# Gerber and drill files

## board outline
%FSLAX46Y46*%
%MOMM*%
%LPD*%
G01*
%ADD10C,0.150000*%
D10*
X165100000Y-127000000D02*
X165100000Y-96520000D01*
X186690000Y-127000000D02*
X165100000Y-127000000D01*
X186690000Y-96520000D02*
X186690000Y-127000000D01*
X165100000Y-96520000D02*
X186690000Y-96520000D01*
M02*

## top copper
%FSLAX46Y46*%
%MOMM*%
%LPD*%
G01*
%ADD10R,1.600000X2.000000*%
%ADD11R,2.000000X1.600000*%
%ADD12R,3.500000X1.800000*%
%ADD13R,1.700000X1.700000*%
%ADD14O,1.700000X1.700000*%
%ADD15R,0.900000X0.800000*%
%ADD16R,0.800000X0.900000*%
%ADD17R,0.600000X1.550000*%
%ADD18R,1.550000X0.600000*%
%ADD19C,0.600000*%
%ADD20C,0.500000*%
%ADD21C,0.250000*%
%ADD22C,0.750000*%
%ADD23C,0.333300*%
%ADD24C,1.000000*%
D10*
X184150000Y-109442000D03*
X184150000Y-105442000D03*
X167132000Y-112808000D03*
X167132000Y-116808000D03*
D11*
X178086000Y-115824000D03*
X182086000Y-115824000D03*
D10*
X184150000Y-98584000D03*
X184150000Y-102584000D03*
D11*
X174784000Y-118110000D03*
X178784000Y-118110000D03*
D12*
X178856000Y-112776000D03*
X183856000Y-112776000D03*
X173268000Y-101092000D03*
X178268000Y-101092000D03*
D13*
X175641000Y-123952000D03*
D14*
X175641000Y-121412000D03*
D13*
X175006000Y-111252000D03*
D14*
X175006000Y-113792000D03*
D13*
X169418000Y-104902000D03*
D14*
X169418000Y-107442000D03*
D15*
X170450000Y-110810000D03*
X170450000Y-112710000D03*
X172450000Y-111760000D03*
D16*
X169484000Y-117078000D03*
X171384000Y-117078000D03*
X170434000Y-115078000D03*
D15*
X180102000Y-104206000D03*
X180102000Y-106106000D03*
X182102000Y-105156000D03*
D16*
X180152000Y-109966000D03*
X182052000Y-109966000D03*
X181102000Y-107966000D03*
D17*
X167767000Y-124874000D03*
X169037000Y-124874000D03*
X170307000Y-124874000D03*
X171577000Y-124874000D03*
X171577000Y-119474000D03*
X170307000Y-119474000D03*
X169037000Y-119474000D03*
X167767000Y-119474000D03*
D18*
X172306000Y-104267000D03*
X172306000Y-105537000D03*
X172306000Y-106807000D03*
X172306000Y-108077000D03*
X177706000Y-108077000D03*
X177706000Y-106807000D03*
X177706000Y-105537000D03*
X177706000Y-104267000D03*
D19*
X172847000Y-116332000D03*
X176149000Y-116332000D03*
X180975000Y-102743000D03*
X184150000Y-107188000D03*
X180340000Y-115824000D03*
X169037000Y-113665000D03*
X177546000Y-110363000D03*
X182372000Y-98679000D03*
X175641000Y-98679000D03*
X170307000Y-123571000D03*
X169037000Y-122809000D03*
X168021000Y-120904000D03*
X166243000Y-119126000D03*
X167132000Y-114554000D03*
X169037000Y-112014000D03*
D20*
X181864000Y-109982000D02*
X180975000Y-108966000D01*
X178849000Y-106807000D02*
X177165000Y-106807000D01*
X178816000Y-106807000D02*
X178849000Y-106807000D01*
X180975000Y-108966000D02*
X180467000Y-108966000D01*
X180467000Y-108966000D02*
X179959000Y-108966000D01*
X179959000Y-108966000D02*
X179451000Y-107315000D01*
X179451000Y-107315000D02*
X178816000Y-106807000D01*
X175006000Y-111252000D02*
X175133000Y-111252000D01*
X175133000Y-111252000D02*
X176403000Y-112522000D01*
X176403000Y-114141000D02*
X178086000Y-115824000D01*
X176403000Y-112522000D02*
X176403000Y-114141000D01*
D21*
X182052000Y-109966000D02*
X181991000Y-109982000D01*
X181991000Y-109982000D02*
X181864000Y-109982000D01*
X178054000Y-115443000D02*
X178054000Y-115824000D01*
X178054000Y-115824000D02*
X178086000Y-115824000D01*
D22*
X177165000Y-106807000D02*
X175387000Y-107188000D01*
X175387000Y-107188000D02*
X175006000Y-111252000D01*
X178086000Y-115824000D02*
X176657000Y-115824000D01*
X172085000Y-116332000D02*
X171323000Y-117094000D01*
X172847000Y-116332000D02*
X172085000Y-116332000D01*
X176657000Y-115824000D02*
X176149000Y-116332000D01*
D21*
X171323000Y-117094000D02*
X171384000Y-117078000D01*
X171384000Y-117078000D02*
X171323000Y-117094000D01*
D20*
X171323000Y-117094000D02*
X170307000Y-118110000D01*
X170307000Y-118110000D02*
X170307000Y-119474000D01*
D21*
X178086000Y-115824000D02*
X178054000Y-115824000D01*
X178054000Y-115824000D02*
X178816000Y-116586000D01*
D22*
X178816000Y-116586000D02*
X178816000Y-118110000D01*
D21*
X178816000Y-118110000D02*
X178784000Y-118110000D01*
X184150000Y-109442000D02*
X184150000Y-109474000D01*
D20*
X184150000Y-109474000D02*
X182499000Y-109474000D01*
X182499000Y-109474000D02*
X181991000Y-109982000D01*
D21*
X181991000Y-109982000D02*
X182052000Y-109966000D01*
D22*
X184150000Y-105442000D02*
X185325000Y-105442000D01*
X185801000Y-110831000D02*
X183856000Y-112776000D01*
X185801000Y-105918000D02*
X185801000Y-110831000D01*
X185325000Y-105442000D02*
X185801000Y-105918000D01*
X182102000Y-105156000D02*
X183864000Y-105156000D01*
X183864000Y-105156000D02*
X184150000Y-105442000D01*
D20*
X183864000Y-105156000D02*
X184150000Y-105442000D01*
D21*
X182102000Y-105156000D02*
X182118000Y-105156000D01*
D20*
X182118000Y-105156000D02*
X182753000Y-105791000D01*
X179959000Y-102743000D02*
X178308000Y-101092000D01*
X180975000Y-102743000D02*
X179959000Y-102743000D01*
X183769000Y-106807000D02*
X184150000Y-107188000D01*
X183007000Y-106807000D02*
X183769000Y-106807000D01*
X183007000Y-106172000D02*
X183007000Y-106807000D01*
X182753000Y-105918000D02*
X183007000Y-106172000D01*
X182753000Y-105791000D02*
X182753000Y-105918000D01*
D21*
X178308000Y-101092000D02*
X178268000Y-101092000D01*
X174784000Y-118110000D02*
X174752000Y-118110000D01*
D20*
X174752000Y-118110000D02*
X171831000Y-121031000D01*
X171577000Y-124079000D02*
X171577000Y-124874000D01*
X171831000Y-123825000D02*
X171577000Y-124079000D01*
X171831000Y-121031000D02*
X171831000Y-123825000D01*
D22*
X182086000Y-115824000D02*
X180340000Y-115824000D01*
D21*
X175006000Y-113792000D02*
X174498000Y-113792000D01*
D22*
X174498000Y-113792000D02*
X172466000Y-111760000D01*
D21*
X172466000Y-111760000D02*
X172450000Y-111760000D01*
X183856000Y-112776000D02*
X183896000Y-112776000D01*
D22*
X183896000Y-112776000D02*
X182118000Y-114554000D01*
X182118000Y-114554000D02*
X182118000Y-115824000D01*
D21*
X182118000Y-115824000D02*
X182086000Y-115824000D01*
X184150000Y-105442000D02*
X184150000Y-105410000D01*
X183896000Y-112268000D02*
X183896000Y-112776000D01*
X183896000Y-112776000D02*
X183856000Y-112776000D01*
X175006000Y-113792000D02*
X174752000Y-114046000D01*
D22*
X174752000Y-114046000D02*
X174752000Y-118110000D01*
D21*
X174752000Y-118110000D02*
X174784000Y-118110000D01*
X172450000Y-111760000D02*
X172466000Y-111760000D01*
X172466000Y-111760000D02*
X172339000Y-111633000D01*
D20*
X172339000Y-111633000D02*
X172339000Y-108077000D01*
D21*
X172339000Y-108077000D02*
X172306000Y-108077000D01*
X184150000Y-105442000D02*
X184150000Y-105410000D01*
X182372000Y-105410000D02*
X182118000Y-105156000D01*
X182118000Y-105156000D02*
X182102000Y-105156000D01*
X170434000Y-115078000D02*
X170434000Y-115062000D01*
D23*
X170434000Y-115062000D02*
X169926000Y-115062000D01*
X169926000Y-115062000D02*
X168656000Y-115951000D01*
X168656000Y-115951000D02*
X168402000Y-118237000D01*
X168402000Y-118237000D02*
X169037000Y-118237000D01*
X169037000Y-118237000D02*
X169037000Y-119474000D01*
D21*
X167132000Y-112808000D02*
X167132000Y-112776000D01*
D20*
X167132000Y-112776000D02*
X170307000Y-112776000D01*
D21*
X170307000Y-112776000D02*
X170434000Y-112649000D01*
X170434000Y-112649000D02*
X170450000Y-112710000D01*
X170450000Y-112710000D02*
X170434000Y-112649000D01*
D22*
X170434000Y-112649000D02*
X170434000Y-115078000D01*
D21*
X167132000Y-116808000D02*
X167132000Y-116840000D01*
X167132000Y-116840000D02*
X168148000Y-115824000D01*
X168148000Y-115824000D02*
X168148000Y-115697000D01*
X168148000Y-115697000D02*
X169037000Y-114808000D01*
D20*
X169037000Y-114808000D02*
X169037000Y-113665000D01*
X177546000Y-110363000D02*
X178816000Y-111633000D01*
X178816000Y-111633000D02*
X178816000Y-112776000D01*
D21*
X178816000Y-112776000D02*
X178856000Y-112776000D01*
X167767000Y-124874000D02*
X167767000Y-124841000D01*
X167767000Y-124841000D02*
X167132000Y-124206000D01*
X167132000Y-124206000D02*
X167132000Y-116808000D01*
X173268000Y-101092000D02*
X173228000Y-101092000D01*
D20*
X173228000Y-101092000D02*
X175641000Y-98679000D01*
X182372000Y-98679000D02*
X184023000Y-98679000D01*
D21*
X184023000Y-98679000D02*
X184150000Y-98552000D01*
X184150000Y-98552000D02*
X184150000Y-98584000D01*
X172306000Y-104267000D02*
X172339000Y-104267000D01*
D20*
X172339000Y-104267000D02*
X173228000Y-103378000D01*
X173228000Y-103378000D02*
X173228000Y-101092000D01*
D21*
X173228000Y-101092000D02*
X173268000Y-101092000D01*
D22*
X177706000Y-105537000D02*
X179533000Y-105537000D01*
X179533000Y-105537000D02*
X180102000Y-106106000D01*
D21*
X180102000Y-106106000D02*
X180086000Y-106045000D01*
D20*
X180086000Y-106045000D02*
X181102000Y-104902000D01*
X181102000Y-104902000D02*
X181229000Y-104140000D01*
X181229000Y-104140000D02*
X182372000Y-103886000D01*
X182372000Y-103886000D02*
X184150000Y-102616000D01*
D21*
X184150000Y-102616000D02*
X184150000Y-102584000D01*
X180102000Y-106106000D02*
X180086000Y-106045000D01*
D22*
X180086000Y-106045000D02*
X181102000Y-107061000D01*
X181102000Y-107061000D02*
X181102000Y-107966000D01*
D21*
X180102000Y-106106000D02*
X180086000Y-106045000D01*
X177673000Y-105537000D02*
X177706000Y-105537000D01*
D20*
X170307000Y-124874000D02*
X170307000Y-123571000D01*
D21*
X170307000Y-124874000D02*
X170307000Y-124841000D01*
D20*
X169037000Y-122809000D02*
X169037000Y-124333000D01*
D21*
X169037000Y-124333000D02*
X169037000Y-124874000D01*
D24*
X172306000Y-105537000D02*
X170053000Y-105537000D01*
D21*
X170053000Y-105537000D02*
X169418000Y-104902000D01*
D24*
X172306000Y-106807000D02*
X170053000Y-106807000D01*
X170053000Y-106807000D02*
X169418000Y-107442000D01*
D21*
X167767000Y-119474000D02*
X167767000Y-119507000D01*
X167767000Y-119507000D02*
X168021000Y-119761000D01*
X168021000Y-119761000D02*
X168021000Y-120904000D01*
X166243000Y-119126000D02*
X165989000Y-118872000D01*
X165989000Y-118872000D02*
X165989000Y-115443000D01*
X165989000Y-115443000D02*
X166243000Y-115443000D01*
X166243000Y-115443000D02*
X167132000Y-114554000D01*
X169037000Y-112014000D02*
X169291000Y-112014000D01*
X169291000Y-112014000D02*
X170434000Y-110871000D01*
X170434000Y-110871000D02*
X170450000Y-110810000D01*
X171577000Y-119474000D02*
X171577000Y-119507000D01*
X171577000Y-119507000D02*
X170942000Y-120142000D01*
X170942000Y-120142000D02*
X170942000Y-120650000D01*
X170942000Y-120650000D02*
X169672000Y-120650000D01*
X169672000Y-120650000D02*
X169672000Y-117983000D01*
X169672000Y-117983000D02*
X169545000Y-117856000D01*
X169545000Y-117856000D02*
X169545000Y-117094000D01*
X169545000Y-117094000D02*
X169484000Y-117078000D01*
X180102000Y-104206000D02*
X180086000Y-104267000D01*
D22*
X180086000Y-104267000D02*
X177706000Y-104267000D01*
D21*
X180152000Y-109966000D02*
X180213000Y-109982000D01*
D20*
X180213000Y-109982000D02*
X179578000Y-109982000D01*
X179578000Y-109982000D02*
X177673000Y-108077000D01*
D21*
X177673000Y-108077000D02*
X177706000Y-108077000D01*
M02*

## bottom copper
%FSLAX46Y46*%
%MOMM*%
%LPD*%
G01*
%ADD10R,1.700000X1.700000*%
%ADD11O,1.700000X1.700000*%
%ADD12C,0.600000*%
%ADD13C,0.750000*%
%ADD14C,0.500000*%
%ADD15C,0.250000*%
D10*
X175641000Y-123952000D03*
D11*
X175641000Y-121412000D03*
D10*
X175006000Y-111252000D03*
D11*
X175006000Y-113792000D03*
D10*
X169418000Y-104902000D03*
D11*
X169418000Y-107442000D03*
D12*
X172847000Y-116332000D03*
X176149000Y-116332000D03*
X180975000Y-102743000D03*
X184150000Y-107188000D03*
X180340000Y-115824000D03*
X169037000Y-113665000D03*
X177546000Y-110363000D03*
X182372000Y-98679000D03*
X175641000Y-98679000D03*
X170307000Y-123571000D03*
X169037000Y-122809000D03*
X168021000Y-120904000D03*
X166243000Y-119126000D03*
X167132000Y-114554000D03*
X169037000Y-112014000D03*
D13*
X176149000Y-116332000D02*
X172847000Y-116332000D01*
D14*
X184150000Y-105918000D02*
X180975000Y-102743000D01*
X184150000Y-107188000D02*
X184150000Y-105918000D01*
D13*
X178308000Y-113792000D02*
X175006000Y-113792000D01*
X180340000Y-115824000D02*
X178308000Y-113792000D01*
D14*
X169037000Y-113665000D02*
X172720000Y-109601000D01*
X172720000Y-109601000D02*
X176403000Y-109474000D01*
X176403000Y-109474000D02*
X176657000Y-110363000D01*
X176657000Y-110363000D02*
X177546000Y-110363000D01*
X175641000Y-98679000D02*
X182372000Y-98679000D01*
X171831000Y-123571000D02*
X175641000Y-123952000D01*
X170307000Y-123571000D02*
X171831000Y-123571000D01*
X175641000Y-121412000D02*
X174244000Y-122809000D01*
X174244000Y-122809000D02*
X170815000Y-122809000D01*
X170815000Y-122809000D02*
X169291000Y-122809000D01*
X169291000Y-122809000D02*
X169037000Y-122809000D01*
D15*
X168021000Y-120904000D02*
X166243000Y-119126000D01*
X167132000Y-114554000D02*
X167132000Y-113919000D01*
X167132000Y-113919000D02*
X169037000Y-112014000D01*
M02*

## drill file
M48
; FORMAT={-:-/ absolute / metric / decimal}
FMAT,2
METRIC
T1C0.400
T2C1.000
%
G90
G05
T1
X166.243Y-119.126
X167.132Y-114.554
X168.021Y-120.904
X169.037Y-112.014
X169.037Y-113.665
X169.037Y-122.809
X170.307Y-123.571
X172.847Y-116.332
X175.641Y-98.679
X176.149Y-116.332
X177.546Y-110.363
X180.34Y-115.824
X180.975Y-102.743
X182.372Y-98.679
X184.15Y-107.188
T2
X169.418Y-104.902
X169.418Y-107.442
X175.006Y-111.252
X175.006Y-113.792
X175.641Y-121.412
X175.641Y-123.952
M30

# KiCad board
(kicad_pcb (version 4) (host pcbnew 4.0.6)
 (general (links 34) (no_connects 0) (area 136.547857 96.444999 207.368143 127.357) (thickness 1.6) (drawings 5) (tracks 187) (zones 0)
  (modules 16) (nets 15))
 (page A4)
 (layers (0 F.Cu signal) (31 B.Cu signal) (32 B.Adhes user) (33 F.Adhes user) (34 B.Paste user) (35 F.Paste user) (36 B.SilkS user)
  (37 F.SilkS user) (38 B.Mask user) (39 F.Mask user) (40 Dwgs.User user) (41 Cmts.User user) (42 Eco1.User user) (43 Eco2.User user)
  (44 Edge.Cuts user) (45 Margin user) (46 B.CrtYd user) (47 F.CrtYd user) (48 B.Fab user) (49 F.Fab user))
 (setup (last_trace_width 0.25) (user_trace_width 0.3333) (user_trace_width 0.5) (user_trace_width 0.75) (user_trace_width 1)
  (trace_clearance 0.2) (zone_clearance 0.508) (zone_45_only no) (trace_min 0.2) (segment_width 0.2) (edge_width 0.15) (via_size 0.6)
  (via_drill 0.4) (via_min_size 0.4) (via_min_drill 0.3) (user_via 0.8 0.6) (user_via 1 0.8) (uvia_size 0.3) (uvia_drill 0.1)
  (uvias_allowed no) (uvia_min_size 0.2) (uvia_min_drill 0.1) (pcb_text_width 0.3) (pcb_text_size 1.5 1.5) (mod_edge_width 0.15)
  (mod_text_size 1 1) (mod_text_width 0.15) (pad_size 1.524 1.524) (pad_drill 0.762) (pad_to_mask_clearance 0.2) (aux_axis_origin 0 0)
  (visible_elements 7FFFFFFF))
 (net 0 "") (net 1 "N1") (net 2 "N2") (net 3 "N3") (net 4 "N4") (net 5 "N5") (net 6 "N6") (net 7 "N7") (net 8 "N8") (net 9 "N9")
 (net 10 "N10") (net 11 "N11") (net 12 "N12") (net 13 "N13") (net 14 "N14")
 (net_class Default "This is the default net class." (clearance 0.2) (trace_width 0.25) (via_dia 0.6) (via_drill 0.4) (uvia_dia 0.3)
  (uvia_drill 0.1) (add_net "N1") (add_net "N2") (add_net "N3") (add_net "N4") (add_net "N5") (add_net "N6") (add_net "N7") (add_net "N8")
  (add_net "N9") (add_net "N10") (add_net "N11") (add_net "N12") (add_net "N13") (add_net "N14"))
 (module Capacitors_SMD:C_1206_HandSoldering (layer F.Cu) (at 184.15 107.442 90)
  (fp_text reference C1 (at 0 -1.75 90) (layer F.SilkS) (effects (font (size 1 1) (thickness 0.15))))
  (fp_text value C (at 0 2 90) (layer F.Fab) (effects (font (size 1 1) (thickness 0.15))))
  (pad 1 smd rect (at -2 0 90) (size 2 1.6) (layers F.Cu F.Paste F.Mask) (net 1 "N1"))
  (pad 2 smd rect (at 2 0 90) (size 2 1.6) (layers F.Cu F.Paste F.Mask) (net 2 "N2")))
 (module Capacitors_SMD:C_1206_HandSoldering (layer F.Cu) (at 167.132 114.808 270)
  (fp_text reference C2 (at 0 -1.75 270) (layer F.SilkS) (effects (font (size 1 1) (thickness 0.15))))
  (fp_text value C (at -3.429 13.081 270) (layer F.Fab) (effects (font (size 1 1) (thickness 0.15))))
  (pad 1 smd rect (at -2 0 270) (size 2 1.6) (layers F.Cu F.Paste F.Mask) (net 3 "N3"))
  (pad 2 smd rect (at 2 0 270) (size 2 1.6) (layers F.Cu F.Paste F.Mask) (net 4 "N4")))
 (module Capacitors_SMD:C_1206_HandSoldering (layer F.Cu) (at 180.086 115.824)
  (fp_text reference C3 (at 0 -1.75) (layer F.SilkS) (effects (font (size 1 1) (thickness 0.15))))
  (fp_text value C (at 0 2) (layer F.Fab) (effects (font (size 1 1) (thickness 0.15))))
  (pad 1 smd rect (at -2 0) (size 2 1.6) (layers F.Cu F.Paste F.Mask) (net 1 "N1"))
  (pad 2 smd rect (at 2 0) (size 2 1.6) (layers F.Cu F.Paste F.Mask) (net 2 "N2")))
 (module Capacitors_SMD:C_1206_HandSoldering (layer F.Cu) (at 184.15 100.584 270)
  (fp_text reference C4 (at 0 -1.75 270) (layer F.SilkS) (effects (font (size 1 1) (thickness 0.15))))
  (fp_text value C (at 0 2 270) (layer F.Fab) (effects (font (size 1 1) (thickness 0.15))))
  (pad 1 smd rect (at -2 0 270) (size 2 1.6) (layers F.Cu F.Paste F.Mask) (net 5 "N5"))
  (pad 2 smd rect (at 2 0 270) (size 2 1.6) (layers F.Cu F.Paste F.Mask) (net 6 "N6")))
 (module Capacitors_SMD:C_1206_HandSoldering (layer F.Cu) (at 176.784 118.11)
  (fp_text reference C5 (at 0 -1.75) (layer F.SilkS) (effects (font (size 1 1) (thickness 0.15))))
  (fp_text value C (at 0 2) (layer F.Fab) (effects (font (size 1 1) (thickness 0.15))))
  (pad 1 smd rect (at -2 0) (size 2 1.6) (layers F.Cu F.Paste F.Mask) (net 2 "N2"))
  (pad 2 smd rect (at 2 0) (size 2 1.6) (layers F.Cu F.Paste F.Mask) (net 1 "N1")))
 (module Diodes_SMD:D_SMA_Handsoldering (layer F.Cu) (at 181.356 112.776)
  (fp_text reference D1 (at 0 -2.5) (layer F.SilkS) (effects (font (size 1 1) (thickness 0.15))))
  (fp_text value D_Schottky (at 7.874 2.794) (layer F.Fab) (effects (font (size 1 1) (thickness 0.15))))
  (pad 1 smd rect (at -2.5 0) (size 3.5 1.8) (layers F.Cu F.Paste F.Mask) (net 4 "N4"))
  (pad 2 smd rect (at 2.5 0) (size 3.5 1.8) (layers F.Cu F.Paste F.Mask) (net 2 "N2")))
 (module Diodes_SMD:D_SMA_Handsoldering (layer F.Cu) (at 175.768 101.092)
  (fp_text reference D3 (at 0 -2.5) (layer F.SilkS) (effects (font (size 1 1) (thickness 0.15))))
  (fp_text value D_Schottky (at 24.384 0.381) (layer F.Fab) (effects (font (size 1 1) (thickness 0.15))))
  (pad 1 smd rect (at -2.5 0) (size 3.5 1.8) (layers F.Cu F.Paste F.Mask) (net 5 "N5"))
  (pad 2 smd rect (at 2.5 0) (size 3.5 1.8) (layers F.Cu F.Paste F.Mask) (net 2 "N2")))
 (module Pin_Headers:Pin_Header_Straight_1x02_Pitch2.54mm (layer F.Cu) (at 175.641 123.952 180)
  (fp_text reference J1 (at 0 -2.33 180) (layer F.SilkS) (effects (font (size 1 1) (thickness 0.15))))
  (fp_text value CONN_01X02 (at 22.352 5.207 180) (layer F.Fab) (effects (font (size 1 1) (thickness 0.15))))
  (pad 1 thru_hole rect (at 0 0 180) (size 1.7 1.7) (drill 1) (layers *.Cu *.Mask) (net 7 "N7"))
  (pad 2 thru_hole oval (at 0 2.54 180) (size 1.7 1.7) (drill 1) (layers *.Cu *.Mask) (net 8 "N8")))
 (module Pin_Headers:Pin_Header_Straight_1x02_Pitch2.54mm (layer F.Cu) (at 175.006 111.252)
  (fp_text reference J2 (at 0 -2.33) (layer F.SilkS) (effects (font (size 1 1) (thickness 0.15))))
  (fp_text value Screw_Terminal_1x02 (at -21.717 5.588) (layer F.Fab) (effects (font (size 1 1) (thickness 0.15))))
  (pad 1 thru_hole rect (at 0 0) (size 1.7 1.7) (drill 1) (layers *.Cu *.Mask) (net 1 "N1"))
  (pad 2 thru_hole oval (at 0 2.54) (size 1.7 1.7) (drill 1) (layers *.Cu *.Mask) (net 2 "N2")))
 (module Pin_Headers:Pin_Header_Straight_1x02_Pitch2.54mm (layer F.Cu) (at 169.418 104.902)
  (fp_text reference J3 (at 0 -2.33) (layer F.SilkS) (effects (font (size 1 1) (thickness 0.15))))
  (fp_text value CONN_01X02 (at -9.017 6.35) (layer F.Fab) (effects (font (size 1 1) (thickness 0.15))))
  (pad 1 thru_hole rect (at 0 0) (size 1.7 1.7) (drill 1) (layers *.Cu *.Mask) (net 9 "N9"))
  (pad 2 thru_hole oval (at 0 2.54) (size 1.7 1.7) (drill 1) (layers *.Cu *.Mask) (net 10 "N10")))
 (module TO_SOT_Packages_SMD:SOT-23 (layer F.Cu) (at 171.45 111.76)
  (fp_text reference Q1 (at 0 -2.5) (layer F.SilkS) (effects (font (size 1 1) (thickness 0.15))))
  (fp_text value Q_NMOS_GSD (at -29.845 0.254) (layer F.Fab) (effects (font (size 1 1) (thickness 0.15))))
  (pad 1 smd rect (at -1 -0.95) (size 0.9 0.8) (layers F.Cu F.Paste F.Mask) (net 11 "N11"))
  (pad 2 smd rect (at -1 0.95) (size 0.9 0.8) (layers F.Cu F.Paste F.Mask) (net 3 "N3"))
  (pad 3 smd rect (at 1 0) (size 0.9 0.8) (layers F.Cu F.Paste F.Mask) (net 2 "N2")))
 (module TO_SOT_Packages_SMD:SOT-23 (layer F.Cu) (at 170.434 116.078 90)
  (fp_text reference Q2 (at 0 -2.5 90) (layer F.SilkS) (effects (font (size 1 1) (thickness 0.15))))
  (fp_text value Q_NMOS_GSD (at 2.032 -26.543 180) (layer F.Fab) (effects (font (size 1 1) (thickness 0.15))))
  (pad 1 smd rect (at -1 -0.95 90) (size 0.9 0.8) (layers F.Cu F.Paste F.Mask) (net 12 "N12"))
  (pad 2 smd rect (at -1 0.95 90) (size 0.9 0.8) (layers F.Cu F.Paste F.Mask) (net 1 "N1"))
  (pad 3 smd rect (at 1 0 90) (size 0.9 0.8) (layers F.Cu F.Paste F.Mask) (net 3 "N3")))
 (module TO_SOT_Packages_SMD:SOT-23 (layer F.Cu) (at 181.102 105.156)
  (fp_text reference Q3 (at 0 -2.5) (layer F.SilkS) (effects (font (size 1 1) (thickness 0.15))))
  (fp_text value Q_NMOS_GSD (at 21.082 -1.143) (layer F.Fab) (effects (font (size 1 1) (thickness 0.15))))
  (pad 1 smd rect (at -1 -0.95) (size 0.9 0.8) (layers F.Cu F.Paste F.Mask) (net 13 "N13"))
  (pad 2 smd rect (at -1 0.95) (size 0.9 0.8) (layers F.Cu F.Paste F.Mask) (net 6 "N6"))
  (pad 3 smd rect (at 1 0) (size 0.9 0.8) (layers F.Cu F.Paste F.Mask) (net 2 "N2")))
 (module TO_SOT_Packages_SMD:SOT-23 (layer F.Cu) (at 181.102 108.966 90)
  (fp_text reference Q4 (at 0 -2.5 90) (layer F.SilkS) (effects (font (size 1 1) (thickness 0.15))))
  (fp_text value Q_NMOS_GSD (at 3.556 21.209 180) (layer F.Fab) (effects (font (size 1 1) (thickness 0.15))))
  (pad 1 smd rect (at -1 -0.95 90) (size 0.9 0.8) (layers F.Cu F.Paste F.Mask) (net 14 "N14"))
  (pad 2 smd rect (at -1 0.95 90) (size 0.9 0.8) (layers F.Cu F.Paste F.Mask) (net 1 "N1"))
  (pad 3 smd rect (at 1 0 90) (size 0.9 0.8) (layers F.Cu F.Paste F.Mask) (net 6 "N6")))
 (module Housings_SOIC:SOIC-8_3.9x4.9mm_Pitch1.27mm (layer F.Cu) (at 169.672 122.174 90)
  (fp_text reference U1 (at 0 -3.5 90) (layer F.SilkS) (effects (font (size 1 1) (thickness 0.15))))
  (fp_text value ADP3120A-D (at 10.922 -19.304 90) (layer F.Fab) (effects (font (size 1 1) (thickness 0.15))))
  (pad 1 smd rect (at -2.7 -1.905 90) (size 1.55 0.6) (layers F.Cu F.Paste F.Mask) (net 4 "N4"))
  (pad 2 smd rect (at -2.7 -0.635 90) (size 1.55 0.6) (layers F.Cu F.Paste F.Mask) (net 8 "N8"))
  (pad 3 smd rect (at -2.7 0.635 90) (size 1.55 0.6) (layers F.Cu F.Paste F.Mask) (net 7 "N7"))
  (pad 4 smd rect (at -2.7 1.905 90) (size 1.55 0.6) (layers F.Cu F.Paste F.Mask) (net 2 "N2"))
  (pad 5 smd rect (at 2.7 1.905 90) (size 1.55 0.6) (layers F.Cu F.Paste F.Mask) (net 12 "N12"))
  (pad 6 smd rect (at 2.7 0.635 90) (size 1.55 0.6) (layers F.Cu F.Paste F.Mask) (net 1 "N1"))
  (pad 7 smd rect (at 2.7 -0.635 90) (size 1.55 0.6) (layers F.Cu F.Paste F.Mask) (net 3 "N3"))
  (pad 8 smd rect (at 2.7 -1.905 90) (size 1.55 0.6) (layers F.Cu F.Paste F.Mask) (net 11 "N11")))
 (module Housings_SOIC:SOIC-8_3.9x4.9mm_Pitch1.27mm (layer F.Cu) (at 175.006 106.172)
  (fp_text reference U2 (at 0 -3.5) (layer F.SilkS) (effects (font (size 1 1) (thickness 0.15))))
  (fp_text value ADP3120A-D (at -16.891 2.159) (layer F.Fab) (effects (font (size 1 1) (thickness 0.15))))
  (pad 1 smd rect (at -2.7 -1.905) (size 1.55 0.6) (layers F.Cu F.Paste F.Mask) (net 5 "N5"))
  (pad 2 smd rect (at -2.7 -0.635) (size 1.55 0.6) (layers F.Cu F.Paste F.Mask) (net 9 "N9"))
  (pad 3 smd rect (at -2.7 0.635) (size 1.55 0.6) (layers F.Cu F.Paste F.Mask) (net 10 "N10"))
  (pad 4 smd rect (at -2.7 1.905) (size 1.55 0.6) (layers F.Cu F.Paste F.Mask) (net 2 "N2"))
  (pad 5 smd rect (at 2.7 1.905) (size 1.55 0.6) (layers F.Cu F.Paste F.Mask) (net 14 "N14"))
  (pad 6 smd rect (at 2.7 0.635) (size 1.55 0.6) (layers F.Cu F.Paste F.Mask) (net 1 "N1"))
  (pad 7 smd rect (at 2.7 -0.635) (size 1.55 0.6) (layers F.Cu F.Paste F.Mask) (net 6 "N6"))
  (pad 8 smd rect (at 2.7 -1.905) (size 1.55 0.6) (layers F.Cu F.Paste F.Mask) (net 13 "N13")))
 (gr_line (start 165.1 127) (end 165.1 96.52) (angle 90) (layer Edge.Cuts) (width 0.15))
 (gr_line (start 186.69 127) (end 165.1 127) (angle 90) (layer Edge.Cuts) (width 0.15))
 (gr_line (start 186.69 96.52) (end 186.69 127) (angle 90) (layer Edge.Cuts) (width 0.15))
 (gr_line (start 165.1 96.52) (end 186.69 96.52) (angle 90) (layer Edge.Cuts) (width 0.15))
 (segment (start 181.864 109.982) (end 180.975 108.966) (width 0.5) (layer F.Cu) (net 1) (status 80000))
 (segment (start 178.849 106.807) (end 177.165 106.807) (width 0.5) (layer F.Cu) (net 1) (status 80000))
 (segment (start 178.816 106.807) (end 178.849 106.807) (width 0.5) (layer F.Cu) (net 1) (status 80000))
 (segment (start 180.975 108.966) (end 180.467 108.966) (width 0.5) (layer F.Cu) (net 1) (status 80000))
 (segment (start 180.467 108.966) (end 179.959 108.966) (width 0.5) (layer F.Cu) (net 1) (status 80000))
 (segment (start 179.959 108.966) (end 179.451 107.315) (width 0.5) (layer F.Cu) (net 1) (status 80000))
 (segment (start 179.451 107.315) (end 178.816 106.807) (width 0.5) (layer F.Cu) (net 1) (status 80000))
 (segment (start 175.006 111.252) (end 175.133 111.252) (width 0.5) (layer F.Cu) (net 1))
 (segment (start 175.133 111.252) (end 176.403 112.522) (width 0.5) (layer F.Cu) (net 1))
 (segment (start 176.403 114.141) (end 178.086 115.824) (width 0.5) (layer F.Cu) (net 1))
 (segment (start 176.403 112.522) (end 176.403 114.141) (width 0.5) (layer F.Cu) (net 1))
 (segment (start 182.052 109.966) (end 181.991 109.982) (width 0.25) (layer F.Cu) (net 1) (status 80000))
 (segment (start 181.991 109.982) (end 181.864 109.982) (width 0.25) (layer F.Cu) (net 1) (status 80000))
 (segment (start 178.054 115.443) (end 178.054 115.824) (width 0.25) (layer F.Cu) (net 1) (status 80000))
 (segment (start 178.054 115.824) (end 178.086 115.824) (width 0.25) (layer F.Cu) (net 1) (status 80000))
 (segment (start 177.165 106.807) (end 175.387 107.188) (width 0.75) (layer F.Cu) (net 1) (status 80000))
 (segment (start 175.387 107.188) (end 175.006 111.252) (width 0.75) (layer F.Cu) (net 1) (status 80000))
 (segment (start 178.086 115.824) (end 176.657 115.824) (width 0.75) (layer F.Cu) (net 1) (status 80000))
 (segment (start 172.085 116.332) (end 171.323 117.094) (width 0.75) (layer F.Cu) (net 1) (status 80000))
 (segment (start 172.847 116.332) (end 172.085 116.332) (width 0.75) (layer F.Cu) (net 1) (status 80000))
 (via (at 172.847 116.332) (size 0.6) (drill 0.4) (layers F.Cu B.Cu) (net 1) (status 80000))
 (segment (start 176.149 116.332) (end 172.847 116.332) (width 0.75) (layer B.Cu) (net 1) (status 80000))
 (via (at 176.149 116.332) (size 0.6) (drill 0.4) (layers F.Cu B.Cu) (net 1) (status 80000))
 (segment (start 176.657 115.824) (end 176.149 116.332) (width 0.75) (layer F.Cu) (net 1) (status 80000))
 (segment (start 171.323 117.094) (end 171.384 117.078) (width 0.25) (layer F.Cu) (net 1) (status 80000))
 (segment (start 171.384 117.078) (end 171.323 117.094) (width 0.25) (layer F.Cu) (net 1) (status 80000))
 (segment (start 171.323 117.094) (end 170.307 118.11) (width 0.5) (layer F.Cu) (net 1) (status 80000))
 (segment (start 170.307 118.11) (end 170.307 119.474) (width 0.5) (layer F.Cu) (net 1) (status 80000))
 (segment (start 178.086 115.824) (end 178.054 115.824) (width 0.25) (layer F.Cu) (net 1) (status 80000))
 (segment (start 178.054 115.824) (end 178.816 116.586) (width 0.25) (layer F.Cu) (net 1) (status 80000))
 (segment (start 178.816 116.586) (end 178.816 118.11) (width 0.75) (layer F.Cu) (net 1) (status 80000))
 (segment (start 178.816 118.11) (end 178.784 118.11) (width 0.25) (layer F.Cu) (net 1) (status 80000))
 (segment (start 184.15 109.442) (end 184.15 109.474) (width 0.25) (layer F.Cu) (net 1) (status 80000))
 (segment (start 184.15 109.474) (end 182.499 109.474) (width 0.5) (layer F.Cu) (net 1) (status 80000))
 (segment (start 182.499 109.474) (end 181.991 109.982) (width 0.5) (layer F.Cu) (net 1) (status 80000))
 (segment (start 181.991 109.982) (end 182.052 109.966) (width 0.25) (layer F.Cu) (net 1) (status 80000))
 (segment (start 184.15 105.442) (end 185.325 105.442) (width 0.75) (layer F.Cu) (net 2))
 (segment (start 185.801 110.831) (end 183.856 112.776) (width 0.75) (layer F.Cu) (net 2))
 (segment (start 185.801 105.918) (end 185.801 110.831) (width 0.75) (layer F.Cu) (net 2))
 (segment (start 185.325 105.442) (end 185.801 105.918) (width 0.75) (layer F.Cu) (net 2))
 (segment (start 182.102 105.156) (end 183.864 105.156) (width 0.75) (layer F.Cu) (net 2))
 (segment (start 183.864 105.156) (end 184.15 105.442) (width 0.75) (layer F.Cu) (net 2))
 (segment (start 183.864 105.156) (end 184.15 105.442) (width 0.5) (layer F.Cu) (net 2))
 (segment (start 182.102 105.156) (end 182.118 105.156) (width 0.25) (layer F.Cu) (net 2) (status 80000))
 (segment (start 182.118 105.156) (end 182.753 105.791) (width 0.5) (layer F.Cu) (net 2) (status 80000))
 (segment (start 179.959 102.743) (end 178.308 101.092) (width 0.5) (layer F.Cu) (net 2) (status 80000))
 (segment (start 180.975 102.743) (end 179.959 102.743) (width 0.5) (layer F.Cu) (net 2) (status 80000))
 (via (at 180.975 102.743) (size 0.6) (drill 0.4) (layers F.Cu B.Cu) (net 2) (status 80000))
 (segment (start 184.15 105.918) (end 180.975 102.743) (width 0.5) (layer B.Cu) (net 2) (status 80000))
 (segment (start 184.15 107.188) (end 184.15 105.918) (width 0.5) (layer B.Cu) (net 2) (status 80000))
 (via (at 184.15 107.188) (size 0.6) (drill 0.4) (layers F.Cu B.Cu) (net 2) (status 80000))
 (segment (start 183.769 106.807) (end 184.15 107.188) (width 0.5) (layer F.Cu) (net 2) (status 80000))
 (segment (start 183.007 106.807) (end 183.769 106.807) (width 0.5) (layer F.Cu) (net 2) (status 80000))
 (segment (start 183.007 106.172) (end 183.007 106.807) (width 0.5) (layer F.Cu) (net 2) (status 80000))
 (segment (start 182.753 105.918) (end 183.007 106.172) (width 0.5) (layer F.Cu) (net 2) (status 80000))
 (segment (start 182.753 105.791) (end 182.753 105.918) (width 0.5) (layer F.Cu) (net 2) (status 80000))
 (segment (start 178.308 101.092) (end 178.268 101.092) (width 0.25) (layer F.Cu) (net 2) (status 80000))
 (segment (start 174.784 118.11) (end 174.752 118.11) (width 0.25) (layer F.Cu) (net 2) (status 80000))
 (segment (start 174.752 118.11) (end 171.831 121.031) (width 0.5) (layer F.Cu) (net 2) (status 80000))
 (segment (start 171.577 124.079) (end 171.577 124.874) (width 0.5) (layer F.Cu) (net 2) (status 80000))
 (segment (start 171.831 123.825) (end 171.577 124.079) (width 0.5) (layer F.Cu) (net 2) (status 80000))
 (segment (start 171.831 121.031) (end 171.831 123.825) (width 0.5) (layer F.Cu) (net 2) (status 80000))
 (segment (start 182.086 115.824) (end 180.34 115.824) (width 0.75) (layer F.Cu) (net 2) (status 80000))
 (segment (start 178.308 113.792) (end 175.006 113.792) (width 0.75) (layer B.Cu) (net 2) (status 80000))
 (segment (start 180.34 115.824) (end 178.308 113.792) (width 0.75) (layer B.Cu) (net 2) (status 80000))
 (via (at 180.34 115.824) (size 0.6) (drill 0.4) (layers F.Cu B.Cu) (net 2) (status 80000))
 (segment (start 175.006 113.792) (end 174.498 113.792) (width 0.25) (layer F.Cu) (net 2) (status 80000))
 (segment (start 174.498 113.792) (end 172.466 111.76) (width 0.75) (layer F.Cu) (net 2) (status 80000))
 (segment (start 172.466 111.76) (end 172.45 111.76) (width 0.25) (layer F.Cu) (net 2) (status 80000))
 (segment (start 183.856 112.776) (end 183.896 112.776) (width 0.25) (layer F.Cu) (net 2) (status 80000))
 (segment (start 183.896 112.776) (end 182.118 114.554) (width 0.75) (layer F.Cu) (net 2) (status 80000))
 (segment (start 182.118 114.554) (end 182.118 115.824) (width 0.75) (layer F.Cu) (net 2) (status 80000))
 (segment (start 182.118 115.824) (end 182.086 115.824) (width 0.25) (layer F.Cu) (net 2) (status 80000))
 (segment (start 184.15 105.442) (end 184.15 105.41) (width 0.25) (layer F.Cu) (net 2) (status 80000))
 (segment (start 183.896 112.268) (end 183.896 112.776) (width 0.25) (layer F.Cu) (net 2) (status 80000))
 (segment (start 183.896 112.776) (end 183.856 112.776) (width 0.25) (layer F.Cu) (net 2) (status 80000))
 (segment (start 175.006 113.792) (end 174.752 114.046) (width 0.25) (layer F.Cu) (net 2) (status 80000))
 (segment (start 174.752 114.046) (end 174.752 118.11) (width 0.75) (layer F.Cu) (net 2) (status 80000))
 (segment (start 174.752 118.11) (end 174.784 118.11) (width 0.25) (layer F.Cu) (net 2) (status 80000))
 (segment (start 172.45 111.76) (end 172.466 111.76) (width 0.25) (layer F.Cu) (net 2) (status 80000))
 (segment (start 172.466 111.76) (end 172.339 111.633) (width 0.25) (layer F.Cu) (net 2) (status 80000))
 (segment (start 172.339 111.633) (end 172.339 108.077) (width 0.5) (layer F.Cu) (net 2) (status 80000))
 (segment (start 172.339 108.077) (end 172.306 108.077) (width 0.25) (layer F.Cu) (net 2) (status 80000))
 (segment (start 184.15 105.442) (end 184.15 105.41) (width 0.25) (layer F.Cu) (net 2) (status 80000))
 (segment (start 182.372 105.41) (end 182.118 105.156) (width 0.25) (layer F.Cu) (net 2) (status 80000))
 (segment (start 182.118 105.156) (end 182.102 105.156) (width 0.25) (layer F.Cu) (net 2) (status 80000))
 (segment (start 170.434 115.078) (end 170.434 115.062) (width 0.25) (layer F.Cu) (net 3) (status 80000))
 (segment (start 170.434 115.062) (end 169.926 115.062) (width 0.3333) (layer F.Cu) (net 3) (status 80000))
 (segment (start 169.926 115.062) (end 168.656 115.951) (width 0.3333) (layer F.Cu) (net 3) (status 80000))
 (segment (start 168.656 115.951) (end 168.402 118.237) (width 0.3333) (layer F.Cu) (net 3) (status 80000))
 (segment (start 168.402 118.237) (end 169.037 118.237) (width 0.3333) (layer F.Cu) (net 3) (status 80000))
 (segment (start 169.037 118.237) (end 169.037 119.474) (width 0.3333) (layer F.Cu) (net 3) (status 80000))
 (segment (start 167.132 112.808) (end 167.132 112.776) (width 0.25) (layer F.Cu) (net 3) (status 80000))
 (segment (start 167.132 112.776) (end 170.307 112.776) (width 0.5) (layer F.Cu) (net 3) (status 80000))
 (segment (start 170.307 112.776) (end 170.434 112.649) (width 0.25) (layer F.Cu) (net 3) (status 80000))
 (segment (start 170.434 112.649) (end 170.45 112.71) (width 0.25) (layer F.Cu) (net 3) (status 80000))
 (segment (start 170.45 112.71) (end 170.434 112.649) (width 0.25) (layer F.Cu) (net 3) (status 80000))
 (segment (start 170.434 112.649) (end 170.434 115.078) (width 0.75) (layer F.Cu) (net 3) (status 80000))
 (segment (start 167.132 116.808) (end 167.132 116.84) (width 0.25) (layer F.Cu) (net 4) (status 80000))
 (segment (start 167.132 116.84) (end 168.148 115.824) (width 0.25) (layer F.Cu) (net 4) (status 80000))
 (segment (start 168.148 115.824) (end 168.148 115.697) (width 0.25) (layer F.Cu) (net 4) (status 80000))
 (segment (start 168.148 115.697) (end 169.037 114.808) (width 0.25) (layer F.Cu) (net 4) (status 80000))
 (segment (start 169.037 114.808) (end 169.037 113.665) (width 0.5) (layer F.Cu) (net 4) (status 80000))
 (via (at 169.037 113.665) (size 0.6) (drill 0.4) (layers F.Cu B.Cu) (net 4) (status 80000))
 (segment (start 169.037 113.665) (end 172.72 109.601) (width 0.5) (layer B.Cu) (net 4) (status 80000))
 (segment (start 172.72 109.601) (end 176.403 109.474) (width 0.5) (layer B.Cu) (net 4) (status 80000))
 (segment (start 176.403 109.474) (end 176.657 110.363) (width 0.5) (layer B.Cu) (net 4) (status 80000))
 (segment (start 176.657 110.363) (end 177.546 110.363) (width 0.5) (layer B.Cu) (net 4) (status 80000))
 (via (at 177.546 110.363) (size 0.6) (drill 0.4) (layers F.Cu B.Cu) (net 4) (status 80000))
 (segment (start 177.546 110.363) (end 178.816 111.633) (width 0.5) (layer F.Cu) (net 4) (status 80000))
 (segment (start 178.816 111.633) (end 178.816 112.776) (width 0.5) (layer F.Cu) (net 4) (status 80000))
 (segment (start 178.816 112.776) (end 178.856 112.776) (width 0.25) (layer F.Cu) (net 4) (status 80000))
 (segment (start 167.767 124.874) (end 167.767 124.841) (width 0.25) (layer F.Cu) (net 4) (status 80000))
 (segment (start 167.767 124.841) (end 167.132 124.206) (width 0.25) (layer F.Cu) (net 4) (status 80000))
 (segment (start 167.132 124.206) (end 167.132 116.808) (width 0.25) (layer F.Cu) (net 4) (status 80000))
 (segment (start 173.268 101.092) (end 173.228 101.092) (width 0.25) (layer F.Cu) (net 5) (status 80000))
 (segment (start 173.228 101.092) (end 175.641 98.679) (width 0.5) (layer F.Cu) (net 5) (status 80000))
 (segment (start 182.372 98.679) (end 184.023 98.679) (width 0.5) (layer F.Cu) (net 5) (status 80000))
 (via (at 182.372 98.679) (size 0.6) (drill 0.4) (layers F.Cu B.Cu) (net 5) (status 80000))
 (segment (start 175.641 98.679) (end 182.372 98.679) (width 0.5) (layer B.Cu) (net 5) (status 80000))
 (via (at 175.641 98.679) (size 0.6) (drill 0.4) (layers F.Cu B.Cu) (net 5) (status 80000))
 (segment (start 184.023 98.679) (end 184.15 98.552) (width 0.25) (layer F.Cu) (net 5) (status 80000))
 (segment (start 184.15 98.552) (end 184.15 98.584) (width 0.25) (layer F.Cu) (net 5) (status 80000))
 (segment (start 172.306 104.267) (end 172.339 104.267) (width 0.25) (layer F.Cu) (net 5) (status 80000))
 (segment (start 172.339 104.267) (end 173.228 103.378) (width 0.5) (layer F.Cu) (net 5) (status 80000))
 (segment (start 173.228 103.378) (end 173.228 101.092) (width 0.5) (layer F.Cu) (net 5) (status 80000))
 (segment (start 173.228 101.092) (end 173.268 101.092) (width 0.25) (layer F.Cu) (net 5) (status 80000))
 (segment (start 177.706 105.537) (end 179.533 105.537) (width 0.75) (layer F.Cu) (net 6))
 (segment (start 179.533 105.537) (end 180.102 106.106) (width 0.75) (layer F.Cu) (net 6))
 (segment (start 180.102 106.106) (end 180.086 106.045) (width 0.25) (layer F.Cu) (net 6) (status 80000))
 (segment (start 180.086 106.045) (end 181.102 104.902) (width 0.5) (layer F.Cu) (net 6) (status 80000))
 (segment (start 181.102 104.902) (end 181.229 104.14) (width 0.5) (layer F.Cu) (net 6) (status 80000))
 (segment (start 181.229 104.14) (end 182.372 103.886) (width 0.5) (layer F.Cu) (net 6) (status 80000))
 (segment (start 182.372 103.886) (end 184.15 102.616) (width 0.5) (layer F.Cu) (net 6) (status 80000))
 (segment (start 184.15 102.616) (end 184.15 102.584) (width 0.25) (layer F.Cu) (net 6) (status 80000))
 (segment (start 180.102 106.106) (end 180.086 106.045) (width 0.25) (layer F.Cu) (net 6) (status 80000))
 (segment (start 180.086 106.045) (end 181.102 107.061) (width 0.75) (layer F.Cu) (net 6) (status 80000))
 (segment (start 181.102 107.061) (end 181.102 107.966) (width 0.75) (layer F.Cu) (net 6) (status 80000))
 (segment (start 180.102 106.106) (end 180.086 106.045) (width 0.25) (layer F.Cu) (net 6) (status 80000))
 (segment (start 177.673 105.537) (end 177.706 105.537) (width 0.25) (layer F.Cu) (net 6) (status 80000))
 (segment (start 170.307 124.874) (end 170.307 123.571) (width 0.5) (layer F.Cu) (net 7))
 (segment (start 171.831 123.571) (end 175.641 123.952) (width 0.5) (layer B.Cu) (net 7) (status 80000))
 (segment (start 170.307 123.571) (end 171.831 123.571) (width 0.5) (layer B.Cu) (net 7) (status 80000))
 (via (at 170.307 123.571) (size 0.6) (drill 0.4) (layers F.Cu B.Cu) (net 7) (status 80000))
 (segment (start 170.307 124.874) (end 170.307 124.841) (width 0.25) (layer F.Cu) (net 7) (status 80000))
 (segment (start 175.641 121.412) (end 174.244 122.809) (width 0.5) (layer B.Cu) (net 8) (status 80000))
 (segment (start 174.244 122.809) (end 170.815 122.809) (width 0.5) (layer B.Cu) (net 8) (status 80000))
 (segment (start 170.815 122.809) (end 169.291 122.809) (width 0.5) (layer B.Cu) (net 8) (status 80000))
 (segment (start 169.291 122.809) (end 169.037 122.809) (width 0.5) (layer B.Cu) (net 8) (status 80000))
 (via (at 169.037 122.809) (size 0.6) (drill 0.4) (layers F.Cu B.Cu) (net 8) (status 80000))
 (segment (start 169.037 122.809) (end 169.037 124.333) (width 0.5) (layer F.Cu) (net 8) (status 80000))
 (segment (start 169.037 124.333) (end 169.037 124.874) (width 0.25) (layer F.Cu) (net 8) (status 80000))
 (segment (start 172.306 105.537) (end 170.053 105.537) (width 1) (layer F.Cu) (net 9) (status 80000))
 (segment (start 170.053 105.537) (end 169.418 104.902) (width 0.25) (layer F.Cu) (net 9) (status 80000))
 (segment (start 172.306 106.807) (end 170.053 106.807) (width 1) (layer F.Cu) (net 10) (status 80000))
 (segment (start 170.053 106.807) (end 169.418 107.442) (width 1) (layer F.Cu) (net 10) (status 80000))
 (segment (start 167.767 119.474) (end 167.767 119.507) (width 0.25) (layer F.Cu) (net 11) (status 80000))
 (segment (start 167.767 119.507) (end 168.021 119.761) (width 0.25) (layer F.Cu) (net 11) (status 80000))
 (segment (start 168.021 119.761) (end 168.021 120.904) (width 0.25) (layer F.Cu) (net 11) (status 80000))
 (via (at 168.021 120.904) (size 0.6) (layers F.Cu B.Cu) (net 11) (status 80000))
 (segment (start 168.021 120.904) (end 166.243 119.126) (width 0.25) (layer B.Cu) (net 11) (status 80000))
 (via (at 166.243 119.126) (size 0.6) (layers F.Cu B.Cu) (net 11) (status 80000))
 (segment (start 166.243 119.126) (end 165.989 118.872) (width 0.25) (layer F.Cu) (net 11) (status 80000))
 (segment (start 165.989 118.872) (end 165.989 115.443) (width 0.25) (layer F.Cu) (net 11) (status 80000))
 (segment (start 165.989 115.443) (end 166.243 115.443) (width 0.25) (layer F.Cu) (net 11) (status 80000))
 (segment (start 166.243 115.443) (end 167.132 114.554) (width 0.25) (layer F.Cu) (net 11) (status 80000))
 (via (at 167.132 114.554) (size 0.6) (layers F.Cu B.Cu) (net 11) (status 80000))
 (segment (start 167.132 114.554) (end 167.132 113.919) (width 0.25) (layer B.Cu) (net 11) (status 80000))
 (segment (start 167.132 113.919) (end 169.037 112.014) (width 0.25) (layer B.Cu) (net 11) (status 80000))
 (via (at 169.037 112.014) (size 0.6) (layers F.Cu B.Cu) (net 11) (status 80000))
 (segment (start 169.037 112.014) (end 169.291 112.014) (width 0.25) (layer F.Cu) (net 11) (status 80000))
 (segment (start 169.291 112.014) (end 170.434 110.871) (width 0.25) (layer F.Cu) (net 11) (status 80000))
 (segment (start 170.434 110.871) (end 170.45 110.81) (width 0.25) (layer F.Cu) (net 11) (status 80000))
 (segment (start 171.577 119.474) (end 171.577 119.507) (width 0.25) (layer F.Cu) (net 12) (status 80000))
 (segment (start 171.577 119.507) (end 170.942 120.142) (width 0.25) (layer F.Cu) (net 12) (status 80000))
 (segment (start 170.942 120.142) (end 170.942 120.65) (width 0.25) (layer F.Cu) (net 12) (status 80000))
 (segment (start 170.942 120.65) (end 169.672 120.65) (width 0.25) (layer F.Cu) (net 12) (status 80000))
 (segment (start 169.672 120.65) (end 169.672 117.983) (width 0.25) (layer F.Cu) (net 12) (status 80000))
 (segment (start 169.672 117.983) (end 169.545 117.856) (width 0.25) (layer F.Cu) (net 12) (status 80000))
 (segment (start 169.545 117.856) (end 169.545 117.094) (width 0.25) (layer F.Cu) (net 12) (status 80000))
 (segment (start 169.545 117.094) (end 169.484 117.078) (width 0.25) (layer F.Cu) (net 12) (status 80000))
 (segment (start 180.102 104.206) (end 180.086 104.267) (width 0.25) (layer F.Cu) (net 13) (status 80000))
 (segment (start 180.086 104.267) (end 177.706 104.267) (width 0.75) (layer F.Cu) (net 13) (status 80000))
 (segment (start 180.152 109.966) (end 180.213 109.982) (width 0.25) (layer F.Cu) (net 14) (status 80000))
 (segment (start 180.213 109.982) (end 179.578 109.982) (width 0.5) (layer F.Cu) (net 14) (status 80000))
 (segment (start 179.578 109.982) (end 177.673 108.077) (width 0.5) (layer F.Cu) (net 14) (status 80000))
 (segment (start 177.673 108.077) (end 177.706 108.077) (width 0.25) (layer F.Cu) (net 14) (status 80000)))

